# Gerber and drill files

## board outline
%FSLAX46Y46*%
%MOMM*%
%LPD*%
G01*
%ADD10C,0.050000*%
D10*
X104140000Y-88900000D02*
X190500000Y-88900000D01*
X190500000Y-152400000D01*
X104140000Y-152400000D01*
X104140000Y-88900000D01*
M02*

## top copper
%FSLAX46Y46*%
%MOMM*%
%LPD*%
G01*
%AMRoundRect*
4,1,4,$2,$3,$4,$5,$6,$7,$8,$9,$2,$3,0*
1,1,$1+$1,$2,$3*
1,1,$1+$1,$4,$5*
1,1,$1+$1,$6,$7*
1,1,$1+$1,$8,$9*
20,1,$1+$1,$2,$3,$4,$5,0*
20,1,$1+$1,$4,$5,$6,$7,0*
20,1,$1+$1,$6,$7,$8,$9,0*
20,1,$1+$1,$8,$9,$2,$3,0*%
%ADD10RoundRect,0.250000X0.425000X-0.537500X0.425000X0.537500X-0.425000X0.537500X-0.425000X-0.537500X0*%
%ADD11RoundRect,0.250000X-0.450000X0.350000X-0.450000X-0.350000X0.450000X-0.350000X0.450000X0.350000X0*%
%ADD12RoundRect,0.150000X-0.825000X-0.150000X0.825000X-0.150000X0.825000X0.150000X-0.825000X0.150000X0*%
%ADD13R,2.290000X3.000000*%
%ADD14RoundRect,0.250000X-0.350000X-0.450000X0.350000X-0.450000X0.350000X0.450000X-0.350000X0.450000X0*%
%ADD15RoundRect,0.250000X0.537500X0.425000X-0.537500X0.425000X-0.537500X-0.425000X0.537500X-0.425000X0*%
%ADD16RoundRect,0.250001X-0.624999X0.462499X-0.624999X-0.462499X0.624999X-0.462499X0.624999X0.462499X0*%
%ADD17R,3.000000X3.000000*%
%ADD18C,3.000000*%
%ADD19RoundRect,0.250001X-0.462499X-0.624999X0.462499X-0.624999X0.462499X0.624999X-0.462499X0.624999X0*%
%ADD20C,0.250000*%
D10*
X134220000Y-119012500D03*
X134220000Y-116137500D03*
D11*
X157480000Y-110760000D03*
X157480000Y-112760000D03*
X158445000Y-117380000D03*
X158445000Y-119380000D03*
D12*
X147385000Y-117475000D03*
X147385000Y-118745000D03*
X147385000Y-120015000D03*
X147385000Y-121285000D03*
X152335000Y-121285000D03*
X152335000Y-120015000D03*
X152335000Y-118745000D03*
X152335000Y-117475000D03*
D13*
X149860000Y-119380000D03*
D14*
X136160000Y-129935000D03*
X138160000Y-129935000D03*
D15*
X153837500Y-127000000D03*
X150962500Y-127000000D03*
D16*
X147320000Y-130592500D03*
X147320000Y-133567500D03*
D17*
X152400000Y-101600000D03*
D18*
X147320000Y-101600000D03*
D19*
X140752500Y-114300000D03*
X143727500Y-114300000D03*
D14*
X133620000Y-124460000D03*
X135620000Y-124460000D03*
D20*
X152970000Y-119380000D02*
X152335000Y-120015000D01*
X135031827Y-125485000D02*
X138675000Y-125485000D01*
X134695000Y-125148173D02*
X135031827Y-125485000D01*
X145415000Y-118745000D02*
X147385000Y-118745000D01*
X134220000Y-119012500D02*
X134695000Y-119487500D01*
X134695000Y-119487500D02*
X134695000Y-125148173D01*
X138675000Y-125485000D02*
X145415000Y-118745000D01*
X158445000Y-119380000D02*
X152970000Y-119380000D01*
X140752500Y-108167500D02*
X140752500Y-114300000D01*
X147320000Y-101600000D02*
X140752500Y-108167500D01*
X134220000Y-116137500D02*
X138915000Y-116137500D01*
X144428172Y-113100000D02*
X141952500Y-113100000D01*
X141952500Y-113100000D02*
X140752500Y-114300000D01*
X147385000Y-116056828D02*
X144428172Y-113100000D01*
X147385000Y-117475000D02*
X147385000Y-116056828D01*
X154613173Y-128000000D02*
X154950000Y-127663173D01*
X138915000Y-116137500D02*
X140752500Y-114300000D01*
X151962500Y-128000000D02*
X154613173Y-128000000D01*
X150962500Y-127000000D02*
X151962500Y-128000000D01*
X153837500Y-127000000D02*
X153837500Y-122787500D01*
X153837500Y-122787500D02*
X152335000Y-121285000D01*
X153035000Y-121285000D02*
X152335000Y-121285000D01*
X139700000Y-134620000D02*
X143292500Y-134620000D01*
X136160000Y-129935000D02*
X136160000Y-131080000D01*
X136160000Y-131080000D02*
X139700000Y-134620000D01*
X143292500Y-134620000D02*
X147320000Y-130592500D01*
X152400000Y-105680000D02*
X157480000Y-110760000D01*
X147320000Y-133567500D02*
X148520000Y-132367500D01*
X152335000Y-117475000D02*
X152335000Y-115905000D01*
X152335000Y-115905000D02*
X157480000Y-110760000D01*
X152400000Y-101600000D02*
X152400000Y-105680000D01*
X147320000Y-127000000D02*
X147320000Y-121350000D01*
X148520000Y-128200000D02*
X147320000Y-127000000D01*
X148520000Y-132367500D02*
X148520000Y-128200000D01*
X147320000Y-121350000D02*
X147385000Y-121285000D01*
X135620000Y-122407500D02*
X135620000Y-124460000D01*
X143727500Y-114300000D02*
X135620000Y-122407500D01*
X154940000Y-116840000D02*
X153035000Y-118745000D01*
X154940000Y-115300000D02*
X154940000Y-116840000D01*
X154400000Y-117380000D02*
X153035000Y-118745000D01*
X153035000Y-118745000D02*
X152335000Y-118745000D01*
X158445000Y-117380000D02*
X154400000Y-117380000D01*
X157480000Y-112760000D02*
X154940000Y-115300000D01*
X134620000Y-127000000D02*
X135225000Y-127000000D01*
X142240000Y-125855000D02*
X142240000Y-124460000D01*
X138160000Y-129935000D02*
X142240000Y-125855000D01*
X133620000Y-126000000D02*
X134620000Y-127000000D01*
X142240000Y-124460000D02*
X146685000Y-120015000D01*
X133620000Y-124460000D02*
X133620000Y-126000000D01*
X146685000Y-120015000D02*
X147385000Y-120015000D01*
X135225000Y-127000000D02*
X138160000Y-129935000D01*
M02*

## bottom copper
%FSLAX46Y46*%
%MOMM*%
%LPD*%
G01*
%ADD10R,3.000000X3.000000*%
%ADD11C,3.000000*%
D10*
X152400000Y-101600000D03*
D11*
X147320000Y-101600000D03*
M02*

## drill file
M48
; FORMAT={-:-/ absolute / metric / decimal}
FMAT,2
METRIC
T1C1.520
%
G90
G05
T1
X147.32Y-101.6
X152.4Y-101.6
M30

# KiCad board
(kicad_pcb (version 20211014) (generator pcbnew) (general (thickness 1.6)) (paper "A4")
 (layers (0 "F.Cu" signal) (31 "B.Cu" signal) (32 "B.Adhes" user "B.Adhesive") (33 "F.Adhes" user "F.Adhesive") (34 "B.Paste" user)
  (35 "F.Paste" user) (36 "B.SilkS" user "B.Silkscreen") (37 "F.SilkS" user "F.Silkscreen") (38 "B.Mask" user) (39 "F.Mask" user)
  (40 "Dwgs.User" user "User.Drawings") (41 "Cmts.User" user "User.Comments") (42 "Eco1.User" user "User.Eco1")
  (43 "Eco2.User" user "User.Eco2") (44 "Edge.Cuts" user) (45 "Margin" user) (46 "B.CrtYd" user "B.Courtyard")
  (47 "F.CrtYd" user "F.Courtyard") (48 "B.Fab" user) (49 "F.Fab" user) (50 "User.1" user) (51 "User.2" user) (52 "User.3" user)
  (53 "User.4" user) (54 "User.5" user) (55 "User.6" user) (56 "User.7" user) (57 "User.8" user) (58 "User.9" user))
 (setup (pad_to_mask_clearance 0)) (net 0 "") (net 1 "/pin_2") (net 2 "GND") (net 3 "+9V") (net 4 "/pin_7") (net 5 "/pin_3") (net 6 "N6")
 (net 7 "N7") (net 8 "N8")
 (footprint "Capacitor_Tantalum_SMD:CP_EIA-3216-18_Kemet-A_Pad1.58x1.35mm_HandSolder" (layer "F.Cu") (at 134.22 117.575 90)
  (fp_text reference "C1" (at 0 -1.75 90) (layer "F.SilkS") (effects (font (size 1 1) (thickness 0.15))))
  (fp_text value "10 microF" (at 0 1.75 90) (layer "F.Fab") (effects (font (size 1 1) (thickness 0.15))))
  (pad "1" smd roundrect (at -1.4375 0 90) (size 1.575 1.35) (layers "F.Cu" "F.Paste" "F.Mask") (roundrect_rratio 0.185185) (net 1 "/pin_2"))
  (pad "2" smd roundrect (at 1.4375 0 90) (size 1.575 1.35) (layers "F.Cu" "F.Paste" "F.Mask") (roundrect_rratio 0.185185) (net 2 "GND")))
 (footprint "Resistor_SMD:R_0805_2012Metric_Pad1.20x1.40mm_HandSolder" (layer "F.Cu") (at 157.48 111.76 -90)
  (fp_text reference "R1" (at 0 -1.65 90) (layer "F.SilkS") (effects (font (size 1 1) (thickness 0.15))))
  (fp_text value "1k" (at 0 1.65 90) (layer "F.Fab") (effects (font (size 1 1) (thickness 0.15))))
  (pad "1" smd roundrect (at -1 0 270) (size 1.2 1.4) (layers "F.Cu" "F.Paste" "F.Mask") (roundrect_rratio 0.208333) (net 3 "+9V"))
  (pad "2" smd roundrect (at 1 0 270) (size 1.2 1.4) (layers "F.Cu" "F.Paste" "F.Mask") (roundrect_rratio 0.208333) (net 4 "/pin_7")))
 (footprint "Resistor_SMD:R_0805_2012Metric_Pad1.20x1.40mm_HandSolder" (layer "F.Cu") (at 158.445 118.38 -90)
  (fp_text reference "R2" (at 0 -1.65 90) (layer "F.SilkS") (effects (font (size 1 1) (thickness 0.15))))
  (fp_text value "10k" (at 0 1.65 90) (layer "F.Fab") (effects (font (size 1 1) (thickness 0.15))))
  (pad "1" smd roundrect (at -1 0 270) (size 1.2 1.4) (layers "F.Cu" "F.Paste" "F.Mask") (roundrect_rratio 0.208333) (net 4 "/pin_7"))
  (pad "2" smd roundrect (at 1 0 270) (size 1.2 1.4) (layers "F.Cu" "F.Paste" "F.Mask") (roundrect_rratio 0.208333) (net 1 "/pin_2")))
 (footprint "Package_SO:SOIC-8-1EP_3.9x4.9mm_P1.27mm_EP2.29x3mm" (layer "F.Cu") (at 149.86 119.38)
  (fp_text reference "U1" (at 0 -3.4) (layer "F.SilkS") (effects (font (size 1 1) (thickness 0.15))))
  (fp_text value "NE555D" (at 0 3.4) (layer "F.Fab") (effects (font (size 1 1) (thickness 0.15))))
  (pad "" smd roundrect (at -0.57 0.75) (size 0.92 1.21) (layers "F.Paste") (roundrect_rratio 0.25))
  (pad "" smd roundrect (at -0.57 -0.75) (size 0.92 1.21) (layers "F.Paste") (roundrect_rratio 0.25))
  (pad "" smd roundrect (at 0.57 -0.75) (size 0.92 1.21) (layers "F.Paste") (roundrect_rratio 0.25))
  (pad "" smd roundrect (at 0.57 0.75) (size 0.92 1.21) (layers "F.Paste") (roundrect_rratio 0.25))
  (pad "1" smd roundrect (at -2.475 -1.905) (size 1.95 0.6) (layers "F.Cu" "F.Paste" "F.Mask") (roundrect_rratio 0.25) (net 2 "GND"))
  (pad "2" smd roundrect (at -2.475 -0.635) (size 1.95 0.6) (layers "F.Cu" "F.Paste" "F.Mask") (roundrect_rratio 0.25) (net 1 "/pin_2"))
  (pad "3" smd roundrect (at -2.475 0.635) (size 1.95 0.6) (layers "F.Cu" "F.Paste" "F.Mask") (roundrect_rratio 0.25) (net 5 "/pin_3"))
  (pad "4" smd roundrect (at -2.475 1.905) (size 1.95 0.6) (layers "F.Cu" "F.Paste" "F.Mask") (roundrect_rratio 0.25) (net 3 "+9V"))
  (pad "5" smd roundrect (at 2.475 1.905) (size 1.95 0.6) (layers "F.Cu" "F.Paste" "F.Mask") (roundrect_rratio 0.25) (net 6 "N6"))
  (pad "6" smd roundrect (at 2.475 0.635) (size 1.95 0.6) (layers "F.Cu" "F.Paste" "F.Mask") (roundrect_rratio 0.25) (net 1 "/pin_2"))
  (pad "7" smd roundrect (at 2.475 -0.635) (size 1.95 0.6) (layers "F.Cu" "F.Paste" "F.Mask") (roundrect_rratio 0.25) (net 4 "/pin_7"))
  (pad "8" smd roundrect (at 2.475 -1.905) (size 1.95 0.6) (layers "F.Cu" "F.Paste" "F.Mask") (roundrect_rratio 0.25) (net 3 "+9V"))
  (pad "9" smd rect (at 0 0) (size 2.29 3) (layers "F.Cu" "F.Mask")))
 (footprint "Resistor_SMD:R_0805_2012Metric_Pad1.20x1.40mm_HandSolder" (layer "F.Cu") (at 137.16 129.935)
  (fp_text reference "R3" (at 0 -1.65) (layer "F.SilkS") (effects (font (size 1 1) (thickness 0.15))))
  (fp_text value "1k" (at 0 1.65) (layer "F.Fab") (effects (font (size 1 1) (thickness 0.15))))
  (pad "1" smd roundrect (at -1 0) (size 1.2 1.4) (layers "F.Cu" "F.Paste" "F.Mask") (roundrect_rratio 0.208333) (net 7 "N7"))
  (pad "2" smd roundrect (at 1 0) (size 1.2 1.4) (layers "F.Cu" "F.Paste" "F.Mask") (roundrect_rratio 0.208333) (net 5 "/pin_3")))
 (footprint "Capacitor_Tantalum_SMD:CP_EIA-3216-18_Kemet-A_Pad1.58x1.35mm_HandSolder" (layer "F.Cu") (at 152.4 127 180)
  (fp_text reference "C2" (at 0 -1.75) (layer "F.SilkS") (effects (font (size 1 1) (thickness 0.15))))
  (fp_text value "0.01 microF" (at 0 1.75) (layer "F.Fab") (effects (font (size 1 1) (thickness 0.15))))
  (pad "1" smd roundrect (at -1.4375 0 180) (size 1.575 1.35) (layers "F.Cu" "F.Paste" "F.Mask") (roundrect_rratio 0.185185) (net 6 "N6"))
  (pad "2" smd roundrect (at 1.4375 0 180) (size 1.575 1.35) (layers "F.Cu" "F.Paste" "F.Mask") (roundrect_rratio 0.185185) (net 2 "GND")))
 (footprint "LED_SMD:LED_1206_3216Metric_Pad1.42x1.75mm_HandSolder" (layer "F.Cu") (at 147.32 132.08 -90)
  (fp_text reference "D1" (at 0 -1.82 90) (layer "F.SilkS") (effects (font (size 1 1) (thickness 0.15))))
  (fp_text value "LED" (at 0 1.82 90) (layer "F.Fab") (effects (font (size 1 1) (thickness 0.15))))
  (pad "1" smd roundrect (at -1.4875 0 270) (size 1.425 1.75) (layers "F.Cu" "F.Paste" "F.Mask") (roundrect_rratio 0.175439) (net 7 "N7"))
  (pad "2" smd roundrect (at 1.4875 0 270) (size 1.425 1.75) (layers "F.Cu" "F.Paste" "F.Mask") (roundrect_rratio 0.175439) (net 3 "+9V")))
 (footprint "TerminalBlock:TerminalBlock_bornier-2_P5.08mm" (layer "F.Cu") (at 152.4 101.6 180)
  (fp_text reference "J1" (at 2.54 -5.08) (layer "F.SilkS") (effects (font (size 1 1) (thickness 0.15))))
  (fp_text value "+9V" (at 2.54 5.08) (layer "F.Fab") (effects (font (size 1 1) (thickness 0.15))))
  (pad "1" thru_hole rect (at 0 0 180) (size 3 3) (drill 1.52) (layers *.Cu *.Mask) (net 3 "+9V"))
  (pad "2" thru_hole circle (at 5.08 0 180) (size 3 3) (drill 1.52) (layers *.Cu *.Mask) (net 2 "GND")))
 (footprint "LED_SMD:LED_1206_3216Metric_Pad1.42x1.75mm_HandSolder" (layer "F.Cu") (at 142.24 114.3)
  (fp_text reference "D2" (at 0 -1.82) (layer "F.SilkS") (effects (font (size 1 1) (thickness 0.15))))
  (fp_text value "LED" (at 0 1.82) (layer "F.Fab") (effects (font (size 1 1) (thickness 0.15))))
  (pad "1" smd roundrect (at -1.4875 0) (size 1.425 1.75) (layers "F.Cu" "F.Paste" "F.Mask") (roundrect_rratio 0.175439) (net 2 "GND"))
  (pad "2" smd roundrect (at 1.4875 0) (size 1.425 1.75) (layers "F.Cu" "F.Paste" "F.Mask") (roundrect_rratio 0.175439) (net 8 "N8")))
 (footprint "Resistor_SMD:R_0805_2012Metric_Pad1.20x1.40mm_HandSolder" (layer "F.Cu") (at 134.62 124.46)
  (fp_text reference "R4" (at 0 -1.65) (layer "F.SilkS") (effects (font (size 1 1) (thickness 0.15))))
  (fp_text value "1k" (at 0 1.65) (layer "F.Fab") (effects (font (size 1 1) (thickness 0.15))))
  (pad "1" smd roundrect (at -1 0) (size 1.2 1.4) (layers "F.Cu" "F.Paste" "F.Mask") (roundrect_rratio 0.208333) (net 5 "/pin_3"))
  (pad "2" smd roundrect (at 1 0) (size 1.2 1.4) (layers "F.Cu" "F.Paste" "F.Mask") (roundrect_rratio 0.208333) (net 8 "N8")))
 (gr_rect (start 104.14 88.9) (end 190.5 152.4) (layer "Edge.Cuts") (width 0.05) (fill none))
 (segment (start 152.97 119.38) (end 152.335 120.015) (width 0.25) (layer "F.Cu") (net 1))
 (segment (start 135.031827 125.485) (end 138.675 125.485) (width 0.25) (layer "F.Cu") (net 1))
 (segment (start 134.695 125.148173) (end 135.031827 125.485) (width 0.25) (layer "F.Cu") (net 1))
 (segment (start 145.415 118.745) (end 147.385 118.745) (width 0.25) (layer "F.Cu") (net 1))
 (segment (start 134.22 119.0125) (end 134.695 119.4875) (width 0.25) (layer "F.Cu") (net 1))
 (segment (start 134.695 119.4875) (end 134.695 125.148173) (width 0.25) (layer "F.Cu") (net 1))
 (segment (start 138.675 125.485) (end 145.415 118.745) (width 0.25) (layer "F.Cu") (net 1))
 (segment (start 158.445 119.38) (end 152.97 119.38) (width 0.25) (layer "F.Cu") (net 1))
 (segment (start 140.7525 108.1675) (end 140.7525 114.3) (width 0.25) (layer "F.Cu") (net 2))
 (segment (start 147.32 101.6) (end 140.7525 108.1675) (width 0.25) (layer "F.Cu") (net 2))
 (segment (start 134.22 116.1375) (end 138.915 116.1375) (width 0.25) (layer "F.Cu") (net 2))
 (segment (start 144.428172 113.1) (end 141.9525 113.1) (width 0.25) (layer "F.Cu") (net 2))
 (segment (start 141.9525 113.1) (end 140.7525 114.3) (width 0.25) (layer "F.Cu") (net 2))
 (segment (start 147.385 116.056828) (end 144.428172 113.1) (width 0.25) (layer "F.Cu") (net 2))
 (segment (start 147.385 117.475) (end 147.385 116.056828) (width 0.25) (layer "F.Cu") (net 2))
 (segment (start 154.613173 128) (end 154.95 127.663173) (width 0.25) (layer "F.Cu") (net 2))
 (segment (start 138.915 116.1375) (end 140.7525 114.3) (width 0.25) (layer "F.Cu") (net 2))
 (segment (start 151.9625 128) (end 154.613173 128) (width 0.25) (layer "F.Cu") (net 2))
 (segment (start 150.9625 127) (end 151.9625 128) (width 0.25) (layer "F.Cu") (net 2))
 (segment (start 153.8375 127) (end 153.8375 122.7875) (width 0.25) (layer "F.Cu") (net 6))
 (segment (start 153.8375 122.7875) (end 152.335 121.285) (width 0.25) (layer "F.Cu") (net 6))
 (segment (start 153.035 121.285) (end 152.335 121.285) (width 0.25) (layer "F.Cu") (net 6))
 (segment (start 139.7 134.62) (end 143.2925 134.62) (width 0.25) (layer "F.Cu") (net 7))
 (segment (start 136.16 129.935) (end 136.16 131.08) (width 0.25) (layer "F.Cu") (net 7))
 (segment (start 136.16 131.08) (end 139.7 134.62) (width 0.25) (layer "F.Cu") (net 7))
 (segment (start 143.2925 134.62) (end 147.32 130.5925) (width 0.25) (layer "F.Cu") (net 7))
 (segment (start 152.4 105.68) (end 157.48 110.76) (width 0.25) (layer "F.Cu") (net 3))
 (segment (start 147.32 133.5675) (end 148.52 132.3675) (width 0.25) (layer "F.Cu") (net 3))
 (segment (start 152.335 117.475) (end 152.335 115.905) (width 0.25) (layer "F.Cu") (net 3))
 (segment (start 152.335 115.905) (end 157.48 110.76) (width 0.25) (layer "F.Cu") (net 3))
 (segment (start 152.4 101.6) (end 152.4 105.68) (width 0.25) (layer "F.Cu") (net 3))
 (segment (start 147.32 127) (end 147.32 121.35) (width 0.25) (layer "F.Cu") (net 3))
 (segment (start 148.52 128.2) (end 147.32 127) (width 0.25) (layer "F.Cu") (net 3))
 (segment (start 148.52 132.3675) (end 148.52 128.2) (width 0.25) (layer "F.Cu") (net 3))
 (segment (start 147.32 121.35) (end 147.385 121.285) (width 0.25) (layer "F.Cu") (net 3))
 (segment (start 135.62 122.4075) (end 135.62 124.46) (width 0.25) (layer "F.Cu") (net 8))
 (segment (start 143.7275 114.3) (end 135.62 122.4075) (width 0.25) (layer "F.Cu") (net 8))
 (segment (start 154.94 116.84) (end 153.035 118.745) (width 0.25) (layer "F.Cu") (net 4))
 (segment (start 154.94 115.3) (end 154.94 116.84) (width 0.25) (layer "F.Cu") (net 4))
 (segment (start 154.4 117.38) (end 153.035 118.745) (width 0.25) (layer "F.Cu") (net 4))
 (segment (start 153.035 118.745) (end 152.335 118.745) (width 0.25) (layer "F.Cu") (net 4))
 (segment (start 158.445 117.38) (end 154.4 117.38) (width 0.25) (layer "F.Cu") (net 4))
 (segment (start 157.48 112.76) (end 154.94 115.3) (width 0.25) (layer "F.Cu") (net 4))
 (segment (start 134.62 127) (end 135.225 127) (width 0.25) (layer "F.Cu") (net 5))
 (segment (start 142.24 125.855) (end 142.24 124.46) (width 0.25) (layer "F.Cu") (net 5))
 (segment (start 138.16 129.935) (end 142.24 125.855) (width 0.25) (layer "F.Cu") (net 5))
 (segment (start 133.62 126) (end 134.62 127) (width 0.25) (layer "F.Cu") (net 5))
 (segment (start 142.24 124.46) (end 146.685 120.015) (width 0.25) (layer "F.Cu") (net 5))
 (segment (start 133.62 124.46) (end 133.62 126) (width 0.25) (layer "F.Cu") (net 5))
 (segment (start 146.685 120.015) (end 147.385 120.015) (width 0.25) (layer "F.Cu") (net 5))
 (segment (start 135.225 127) (end 138.16 129.935) (width 0.25) (layer "F.Cu") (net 5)))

